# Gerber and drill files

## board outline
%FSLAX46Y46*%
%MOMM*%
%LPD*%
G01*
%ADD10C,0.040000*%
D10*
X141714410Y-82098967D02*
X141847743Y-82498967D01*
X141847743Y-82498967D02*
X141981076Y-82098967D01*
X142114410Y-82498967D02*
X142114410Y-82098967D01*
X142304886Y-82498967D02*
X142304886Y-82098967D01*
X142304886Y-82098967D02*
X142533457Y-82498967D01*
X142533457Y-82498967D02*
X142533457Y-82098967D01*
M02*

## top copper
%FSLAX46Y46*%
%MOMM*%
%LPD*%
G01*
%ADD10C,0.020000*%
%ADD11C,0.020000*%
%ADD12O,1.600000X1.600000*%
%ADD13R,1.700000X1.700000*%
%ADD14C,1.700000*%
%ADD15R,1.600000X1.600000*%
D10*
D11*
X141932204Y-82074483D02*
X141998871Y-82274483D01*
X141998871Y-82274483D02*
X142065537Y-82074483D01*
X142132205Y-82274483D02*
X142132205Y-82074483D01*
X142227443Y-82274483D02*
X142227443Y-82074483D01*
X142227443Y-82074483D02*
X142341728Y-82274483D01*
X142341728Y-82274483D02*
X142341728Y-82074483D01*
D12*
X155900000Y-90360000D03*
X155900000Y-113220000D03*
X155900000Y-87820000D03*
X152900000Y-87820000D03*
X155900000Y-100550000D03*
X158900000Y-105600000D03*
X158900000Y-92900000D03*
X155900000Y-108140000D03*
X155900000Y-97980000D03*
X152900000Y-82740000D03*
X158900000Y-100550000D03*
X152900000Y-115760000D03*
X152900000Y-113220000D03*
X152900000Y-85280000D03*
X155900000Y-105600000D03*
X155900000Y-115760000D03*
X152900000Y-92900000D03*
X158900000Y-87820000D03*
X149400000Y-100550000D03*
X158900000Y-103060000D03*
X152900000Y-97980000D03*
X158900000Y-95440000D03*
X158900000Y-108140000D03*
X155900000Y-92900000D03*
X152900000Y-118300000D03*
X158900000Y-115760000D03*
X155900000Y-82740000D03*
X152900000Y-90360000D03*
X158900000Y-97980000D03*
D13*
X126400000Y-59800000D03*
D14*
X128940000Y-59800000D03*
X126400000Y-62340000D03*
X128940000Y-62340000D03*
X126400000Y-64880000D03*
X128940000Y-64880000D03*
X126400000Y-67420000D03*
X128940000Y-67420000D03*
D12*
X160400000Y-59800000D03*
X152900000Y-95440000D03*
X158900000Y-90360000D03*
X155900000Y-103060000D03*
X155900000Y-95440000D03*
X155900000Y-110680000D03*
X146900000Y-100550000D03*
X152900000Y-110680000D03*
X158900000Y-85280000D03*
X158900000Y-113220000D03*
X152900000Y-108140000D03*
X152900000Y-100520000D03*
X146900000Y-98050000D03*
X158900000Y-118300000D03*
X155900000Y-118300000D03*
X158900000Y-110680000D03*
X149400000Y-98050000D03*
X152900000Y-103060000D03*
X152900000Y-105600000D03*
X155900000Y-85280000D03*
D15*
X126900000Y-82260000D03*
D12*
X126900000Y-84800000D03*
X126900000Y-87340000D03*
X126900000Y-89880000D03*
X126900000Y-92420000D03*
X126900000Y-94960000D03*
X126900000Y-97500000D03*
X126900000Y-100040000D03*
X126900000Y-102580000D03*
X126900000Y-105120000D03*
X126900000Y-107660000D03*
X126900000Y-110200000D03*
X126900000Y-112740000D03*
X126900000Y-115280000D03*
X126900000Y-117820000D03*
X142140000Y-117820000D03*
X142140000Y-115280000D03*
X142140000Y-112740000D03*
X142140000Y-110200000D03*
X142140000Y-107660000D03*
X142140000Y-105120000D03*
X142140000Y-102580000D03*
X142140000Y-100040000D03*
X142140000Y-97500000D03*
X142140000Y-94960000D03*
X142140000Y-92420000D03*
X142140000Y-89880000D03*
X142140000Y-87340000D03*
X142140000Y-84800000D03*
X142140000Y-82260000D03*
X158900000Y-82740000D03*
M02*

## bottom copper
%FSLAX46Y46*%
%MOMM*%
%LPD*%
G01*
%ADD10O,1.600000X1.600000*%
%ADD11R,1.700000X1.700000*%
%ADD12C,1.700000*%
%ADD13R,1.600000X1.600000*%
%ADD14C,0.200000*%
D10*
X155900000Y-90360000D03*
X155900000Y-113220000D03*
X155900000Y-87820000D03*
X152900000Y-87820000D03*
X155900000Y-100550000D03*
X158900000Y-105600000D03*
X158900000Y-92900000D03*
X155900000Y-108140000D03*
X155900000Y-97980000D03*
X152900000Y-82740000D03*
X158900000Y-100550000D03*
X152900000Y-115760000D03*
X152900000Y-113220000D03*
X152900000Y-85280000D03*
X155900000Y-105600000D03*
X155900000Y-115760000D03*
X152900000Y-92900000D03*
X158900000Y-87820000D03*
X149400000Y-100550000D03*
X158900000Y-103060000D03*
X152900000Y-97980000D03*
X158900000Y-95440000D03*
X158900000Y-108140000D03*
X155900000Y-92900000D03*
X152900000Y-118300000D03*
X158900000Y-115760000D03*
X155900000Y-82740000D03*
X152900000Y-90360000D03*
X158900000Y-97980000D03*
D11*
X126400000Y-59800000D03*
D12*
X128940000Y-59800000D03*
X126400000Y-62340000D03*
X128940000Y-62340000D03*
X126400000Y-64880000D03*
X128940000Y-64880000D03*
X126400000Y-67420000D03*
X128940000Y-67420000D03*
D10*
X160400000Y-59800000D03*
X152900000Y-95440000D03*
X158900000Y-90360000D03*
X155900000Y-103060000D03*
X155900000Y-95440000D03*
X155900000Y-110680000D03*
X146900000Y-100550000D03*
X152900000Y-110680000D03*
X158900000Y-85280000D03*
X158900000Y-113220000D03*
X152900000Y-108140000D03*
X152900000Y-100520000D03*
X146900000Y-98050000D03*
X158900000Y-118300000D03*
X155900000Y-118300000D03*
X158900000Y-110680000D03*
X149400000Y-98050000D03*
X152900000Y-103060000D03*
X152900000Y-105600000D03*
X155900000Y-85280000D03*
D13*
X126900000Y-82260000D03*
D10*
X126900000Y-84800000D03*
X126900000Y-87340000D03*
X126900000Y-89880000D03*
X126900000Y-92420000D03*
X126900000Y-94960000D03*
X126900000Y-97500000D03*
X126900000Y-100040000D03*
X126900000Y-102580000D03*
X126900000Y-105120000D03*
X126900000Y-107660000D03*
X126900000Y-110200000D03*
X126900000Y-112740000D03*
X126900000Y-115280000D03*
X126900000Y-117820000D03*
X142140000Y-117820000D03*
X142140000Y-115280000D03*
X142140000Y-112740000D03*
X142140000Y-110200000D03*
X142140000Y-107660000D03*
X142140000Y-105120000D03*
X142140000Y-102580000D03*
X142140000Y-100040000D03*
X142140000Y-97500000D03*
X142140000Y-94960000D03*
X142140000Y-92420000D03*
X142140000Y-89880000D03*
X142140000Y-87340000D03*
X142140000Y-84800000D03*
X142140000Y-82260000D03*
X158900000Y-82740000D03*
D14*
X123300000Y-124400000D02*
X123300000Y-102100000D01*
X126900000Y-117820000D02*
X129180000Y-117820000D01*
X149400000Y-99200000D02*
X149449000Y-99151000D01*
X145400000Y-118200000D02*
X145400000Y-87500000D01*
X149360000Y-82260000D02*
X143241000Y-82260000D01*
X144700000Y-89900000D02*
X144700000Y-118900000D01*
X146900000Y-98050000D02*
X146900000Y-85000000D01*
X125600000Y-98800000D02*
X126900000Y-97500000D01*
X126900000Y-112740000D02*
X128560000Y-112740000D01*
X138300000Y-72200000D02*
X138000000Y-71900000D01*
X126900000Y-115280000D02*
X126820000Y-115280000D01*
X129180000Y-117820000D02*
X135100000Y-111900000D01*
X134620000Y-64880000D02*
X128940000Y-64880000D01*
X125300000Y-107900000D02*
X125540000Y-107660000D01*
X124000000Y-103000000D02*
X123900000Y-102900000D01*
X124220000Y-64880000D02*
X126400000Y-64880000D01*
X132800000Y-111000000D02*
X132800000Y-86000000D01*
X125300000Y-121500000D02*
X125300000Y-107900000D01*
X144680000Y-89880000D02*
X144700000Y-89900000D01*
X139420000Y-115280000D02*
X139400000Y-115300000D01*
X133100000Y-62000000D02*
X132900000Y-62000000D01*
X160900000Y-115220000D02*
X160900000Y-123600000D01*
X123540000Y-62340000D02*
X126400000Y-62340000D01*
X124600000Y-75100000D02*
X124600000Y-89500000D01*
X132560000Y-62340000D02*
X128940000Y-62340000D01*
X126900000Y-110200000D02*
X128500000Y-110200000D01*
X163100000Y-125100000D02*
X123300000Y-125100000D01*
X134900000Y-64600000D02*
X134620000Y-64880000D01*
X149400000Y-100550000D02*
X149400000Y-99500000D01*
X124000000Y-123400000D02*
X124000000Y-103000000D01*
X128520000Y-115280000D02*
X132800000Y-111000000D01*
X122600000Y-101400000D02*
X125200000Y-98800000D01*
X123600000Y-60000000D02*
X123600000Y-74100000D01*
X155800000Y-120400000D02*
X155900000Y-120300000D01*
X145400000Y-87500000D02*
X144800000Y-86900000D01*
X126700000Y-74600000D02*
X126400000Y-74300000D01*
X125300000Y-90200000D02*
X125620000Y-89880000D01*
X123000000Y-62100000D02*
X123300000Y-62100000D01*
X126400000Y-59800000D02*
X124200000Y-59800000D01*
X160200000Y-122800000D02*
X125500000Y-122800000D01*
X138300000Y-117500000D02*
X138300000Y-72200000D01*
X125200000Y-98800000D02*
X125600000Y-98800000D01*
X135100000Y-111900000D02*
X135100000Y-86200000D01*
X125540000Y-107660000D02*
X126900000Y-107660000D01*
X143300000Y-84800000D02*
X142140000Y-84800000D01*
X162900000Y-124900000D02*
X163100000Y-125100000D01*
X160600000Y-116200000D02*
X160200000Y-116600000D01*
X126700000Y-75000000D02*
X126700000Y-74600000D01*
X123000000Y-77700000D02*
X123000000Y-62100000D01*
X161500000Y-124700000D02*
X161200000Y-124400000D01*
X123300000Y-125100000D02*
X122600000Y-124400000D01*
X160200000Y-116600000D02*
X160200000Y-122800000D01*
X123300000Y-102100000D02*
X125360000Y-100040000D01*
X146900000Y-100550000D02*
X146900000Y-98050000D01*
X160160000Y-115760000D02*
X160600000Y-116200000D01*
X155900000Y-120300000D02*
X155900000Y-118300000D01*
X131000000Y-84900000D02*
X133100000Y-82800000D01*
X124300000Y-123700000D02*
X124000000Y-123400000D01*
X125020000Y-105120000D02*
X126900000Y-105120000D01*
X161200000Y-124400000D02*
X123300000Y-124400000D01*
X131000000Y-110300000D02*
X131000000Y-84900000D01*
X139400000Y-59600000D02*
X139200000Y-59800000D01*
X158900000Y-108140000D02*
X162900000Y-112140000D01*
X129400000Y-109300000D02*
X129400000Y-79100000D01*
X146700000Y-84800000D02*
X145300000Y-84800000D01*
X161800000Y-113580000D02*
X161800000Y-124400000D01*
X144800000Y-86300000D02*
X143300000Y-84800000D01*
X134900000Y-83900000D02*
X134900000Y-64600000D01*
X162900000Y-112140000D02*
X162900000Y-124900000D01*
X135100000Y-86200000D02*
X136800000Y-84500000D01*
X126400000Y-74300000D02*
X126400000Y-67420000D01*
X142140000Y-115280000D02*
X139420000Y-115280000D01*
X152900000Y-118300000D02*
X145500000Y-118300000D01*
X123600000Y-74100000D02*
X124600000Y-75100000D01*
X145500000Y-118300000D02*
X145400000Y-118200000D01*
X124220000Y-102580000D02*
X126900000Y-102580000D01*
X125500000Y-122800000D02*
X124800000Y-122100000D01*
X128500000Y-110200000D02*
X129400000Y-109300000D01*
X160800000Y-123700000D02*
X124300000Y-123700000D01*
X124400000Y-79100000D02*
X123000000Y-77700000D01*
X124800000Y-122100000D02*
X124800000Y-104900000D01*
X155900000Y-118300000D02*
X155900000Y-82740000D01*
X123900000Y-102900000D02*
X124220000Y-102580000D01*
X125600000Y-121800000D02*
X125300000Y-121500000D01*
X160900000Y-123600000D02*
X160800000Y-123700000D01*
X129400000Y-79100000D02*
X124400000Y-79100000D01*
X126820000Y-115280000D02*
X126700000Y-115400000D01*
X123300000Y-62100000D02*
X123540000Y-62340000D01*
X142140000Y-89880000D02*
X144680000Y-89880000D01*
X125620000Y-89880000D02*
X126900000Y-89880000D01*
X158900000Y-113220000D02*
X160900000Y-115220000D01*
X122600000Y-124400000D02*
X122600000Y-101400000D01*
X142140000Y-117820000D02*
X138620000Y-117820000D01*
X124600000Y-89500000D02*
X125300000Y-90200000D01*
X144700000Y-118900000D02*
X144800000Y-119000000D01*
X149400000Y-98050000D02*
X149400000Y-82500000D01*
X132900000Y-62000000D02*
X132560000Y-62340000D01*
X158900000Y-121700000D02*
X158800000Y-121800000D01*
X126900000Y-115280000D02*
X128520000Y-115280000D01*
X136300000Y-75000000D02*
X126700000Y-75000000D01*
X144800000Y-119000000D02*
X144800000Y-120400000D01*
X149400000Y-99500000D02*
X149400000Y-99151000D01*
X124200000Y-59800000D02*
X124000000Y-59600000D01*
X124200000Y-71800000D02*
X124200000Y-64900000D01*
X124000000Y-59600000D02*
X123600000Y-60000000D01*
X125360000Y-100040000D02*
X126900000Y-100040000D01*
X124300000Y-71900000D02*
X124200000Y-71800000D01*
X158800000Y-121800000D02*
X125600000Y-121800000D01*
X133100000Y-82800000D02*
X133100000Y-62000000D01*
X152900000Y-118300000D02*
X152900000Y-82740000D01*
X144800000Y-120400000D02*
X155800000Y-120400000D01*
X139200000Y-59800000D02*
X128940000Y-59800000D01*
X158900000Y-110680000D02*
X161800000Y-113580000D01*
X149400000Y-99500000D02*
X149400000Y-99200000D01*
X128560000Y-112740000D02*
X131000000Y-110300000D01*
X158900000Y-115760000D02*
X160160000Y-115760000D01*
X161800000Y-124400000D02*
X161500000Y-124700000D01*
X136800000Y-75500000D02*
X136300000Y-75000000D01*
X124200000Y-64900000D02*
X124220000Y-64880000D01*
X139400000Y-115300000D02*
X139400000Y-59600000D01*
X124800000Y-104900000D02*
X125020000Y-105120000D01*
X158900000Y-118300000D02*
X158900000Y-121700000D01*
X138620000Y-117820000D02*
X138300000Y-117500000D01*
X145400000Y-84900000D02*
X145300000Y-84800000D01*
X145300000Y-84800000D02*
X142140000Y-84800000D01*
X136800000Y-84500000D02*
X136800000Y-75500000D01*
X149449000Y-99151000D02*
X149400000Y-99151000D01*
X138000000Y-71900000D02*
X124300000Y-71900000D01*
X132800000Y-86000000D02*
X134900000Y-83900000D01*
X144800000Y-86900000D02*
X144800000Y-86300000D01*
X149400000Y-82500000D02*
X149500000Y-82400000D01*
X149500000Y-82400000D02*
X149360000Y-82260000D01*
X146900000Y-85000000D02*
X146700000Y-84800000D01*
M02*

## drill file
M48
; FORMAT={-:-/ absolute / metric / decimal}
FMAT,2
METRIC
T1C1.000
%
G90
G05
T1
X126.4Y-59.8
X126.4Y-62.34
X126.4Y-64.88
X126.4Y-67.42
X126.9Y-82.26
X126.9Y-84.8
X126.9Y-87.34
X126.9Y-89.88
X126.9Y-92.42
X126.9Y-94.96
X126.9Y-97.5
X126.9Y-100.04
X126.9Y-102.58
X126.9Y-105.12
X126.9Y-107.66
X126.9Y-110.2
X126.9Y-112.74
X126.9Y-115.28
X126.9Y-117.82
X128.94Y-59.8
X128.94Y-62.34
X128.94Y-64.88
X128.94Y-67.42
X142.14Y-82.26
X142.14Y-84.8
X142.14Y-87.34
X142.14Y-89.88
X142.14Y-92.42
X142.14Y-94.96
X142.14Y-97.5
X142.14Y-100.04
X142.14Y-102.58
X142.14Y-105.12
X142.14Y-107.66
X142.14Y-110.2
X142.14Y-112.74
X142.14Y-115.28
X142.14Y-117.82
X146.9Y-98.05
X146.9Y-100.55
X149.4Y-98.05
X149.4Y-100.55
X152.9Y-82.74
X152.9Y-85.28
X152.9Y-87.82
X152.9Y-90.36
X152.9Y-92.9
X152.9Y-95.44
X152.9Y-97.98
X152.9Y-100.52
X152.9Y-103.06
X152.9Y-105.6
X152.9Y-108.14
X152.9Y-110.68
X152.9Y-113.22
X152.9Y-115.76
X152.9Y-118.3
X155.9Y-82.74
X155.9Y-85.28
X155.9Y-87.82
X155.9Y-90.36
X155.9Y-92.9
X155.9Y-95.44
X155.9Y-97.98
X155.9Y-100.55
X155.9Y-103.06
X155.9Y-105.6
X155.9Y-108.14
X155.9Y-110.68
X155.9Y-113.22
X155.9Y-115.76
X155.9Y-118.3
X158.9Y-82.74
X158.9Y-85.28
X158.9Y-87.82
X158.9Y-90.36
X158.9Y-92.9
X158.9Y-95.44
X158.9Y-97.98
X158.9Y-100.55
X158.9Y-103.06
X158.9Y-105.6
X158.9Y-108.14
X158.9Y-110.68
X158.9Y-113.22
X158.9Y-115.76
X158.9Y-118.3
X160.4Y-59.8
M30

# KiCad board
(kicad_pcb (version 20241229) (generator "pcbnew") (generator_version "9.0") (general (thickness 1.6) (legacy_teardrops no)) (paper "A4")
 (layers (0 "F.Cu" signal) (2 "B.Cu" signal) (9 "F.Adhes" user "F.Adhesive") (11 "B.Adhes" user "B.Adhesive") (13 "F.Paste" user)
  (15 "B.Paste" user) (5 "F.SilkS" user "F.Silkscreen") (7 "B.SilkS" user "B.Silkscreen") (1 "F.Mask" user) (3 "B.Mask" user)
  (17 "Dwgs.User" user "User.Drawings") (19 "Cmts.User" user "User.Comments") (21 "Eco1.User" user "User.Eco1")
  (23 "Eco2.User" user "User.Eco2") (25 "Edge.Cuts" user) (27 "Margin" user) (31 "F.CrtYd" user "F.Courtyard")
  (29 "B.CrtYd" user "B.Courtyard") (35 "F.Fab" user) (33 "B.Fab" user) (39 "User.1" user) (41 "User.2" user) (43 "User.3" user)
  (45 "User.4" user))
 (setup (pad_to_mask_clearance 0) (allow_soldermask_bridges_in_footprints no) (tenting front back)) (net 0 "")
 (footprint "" (layer "F.Cu") (at 155.9 90.36)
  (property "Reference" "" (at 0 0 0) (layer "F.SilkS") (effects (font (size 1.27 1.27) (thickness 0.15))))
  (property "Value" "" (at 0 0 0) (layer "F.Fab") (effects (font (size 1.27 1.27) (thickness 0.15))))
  (pad "27" thru_hole oval (at 0 0) (size 1.6 1.6) (drill 1) (layers "*.Cu" "*.Mask") (remove_unused_layers no)))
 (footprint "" (layer "F.Cu") (at 155.9 113.22)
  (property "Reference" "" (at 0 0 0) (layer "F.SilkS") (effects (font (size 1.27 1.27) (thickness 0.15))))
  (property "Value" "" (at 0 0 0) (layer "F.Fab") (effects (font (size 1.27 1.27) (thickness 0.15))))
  (pad "18" thru_hole oval (at 0 0) (size 1.6 1.6) (drill 1) (layers "*.Cu" "*.Mask") (remove_unused_layers no)))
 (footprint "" (layer "F.Cu") (at 155.9 87.82)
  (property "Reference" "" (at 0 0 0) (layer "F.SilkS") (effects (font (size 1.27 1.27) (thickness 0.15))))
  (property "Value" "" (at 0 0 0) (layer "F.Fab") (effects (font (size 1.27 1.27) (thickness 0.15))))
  (pad "28" thru_hole oval (at 0 0) (size 1.6 1.6) (drill 1) (layers "*.Cu" "*.Mask") (remove_unused_layers no)))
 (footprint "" (layer "F.Cu") (at 152.9 87.82)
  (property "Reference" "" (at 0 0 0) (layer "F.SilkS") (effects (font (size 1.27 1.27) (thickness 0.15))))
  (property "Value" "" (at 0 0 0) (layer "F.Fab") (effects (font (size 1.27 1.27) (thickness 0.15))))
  (pad "28" thru_hole oval (at 0 0) (size 1.6 1.6) (drill 1) (layers "*.Cu" "*.Mask") (remove_unused_layers no)))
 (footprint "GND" (layer "F.Cu") (at 155.9 100.55)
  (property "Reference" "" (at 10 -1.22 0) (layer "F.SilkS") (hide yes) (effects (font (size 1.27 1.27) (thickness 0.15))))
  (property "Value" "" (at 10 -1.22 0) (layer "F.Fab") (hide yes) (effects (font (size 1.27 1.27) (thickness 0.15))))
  (pad "23" thru_hole oval (at 0 0) (size 1.6 1.6) (drill 1) (layers "*.Cu" "*.Mask") (remove_unused_layers no)))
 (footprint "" (layer "F.Cu") (at 158.9 105.6)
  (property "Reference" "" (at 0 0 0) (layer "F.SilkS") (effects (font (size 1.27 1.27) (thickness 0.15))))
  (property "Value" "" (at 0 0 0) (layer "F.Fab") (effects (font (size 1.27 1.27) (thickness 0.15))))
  (pad "21" thru_hole oval (at 0 0) (size 1.6 1.6) (drill 1) (layers "*.Cu" "*.Mask") (remove_unused_layers no)))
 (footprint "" (layer "F.Cu") (at 158.9 92.9)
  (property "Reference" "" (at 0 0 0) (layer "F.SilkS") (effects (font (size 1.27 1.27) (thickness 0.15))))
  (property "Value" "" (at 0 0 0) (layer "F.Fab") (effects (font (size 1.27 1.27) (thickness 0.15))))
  (pad "26" thru_hole oval (at 0 0) (size 1.6 1.6) (drill 1) (layers "*.Cu" "*.Mask") (remove_unused_layers no)))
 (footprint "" (layer "F.Cu") (at 155.9 108.14)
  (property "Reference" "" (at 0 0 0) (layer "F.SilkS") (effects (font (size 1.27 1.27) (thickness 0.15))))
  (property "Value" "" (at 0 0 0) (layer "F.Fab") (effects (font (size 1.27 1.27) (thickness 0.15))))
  (pad "20" thru_hole oval (at 0 0) (size 1.6 1.6) (drill 1) (layers "*.Cu" "*.Mask") (remove_unused_layers no)))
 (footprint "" (layer "F.Cu") (at 155.9 97.98)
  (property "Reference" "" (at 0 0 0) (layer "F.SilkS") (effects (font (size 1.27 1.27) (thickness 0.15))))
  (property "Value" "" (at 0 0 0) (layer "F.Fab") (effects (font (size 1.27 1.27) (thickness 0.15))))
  (pad "24" thru_hole oval (at 0 0) (size 1.6 1.6) (drill 1) (layers "*.Cu" "*.Mask") (remove_unused_layers no)))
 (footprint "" (layer "F.Cu") (at 152.9 82.74)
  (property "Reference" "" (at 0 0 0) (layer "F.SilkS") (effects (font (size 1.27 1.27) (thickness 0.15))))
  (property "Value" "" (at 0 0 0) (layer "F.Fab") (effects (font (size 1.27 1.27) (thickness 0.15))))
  (pad "30" thru_hole oval (at 0 0) (size 1.6 1.6) (drill 1) (layers "*.Cu" "*.Mask") (remove_unused_layers no)))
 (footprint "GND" (layer "F.Cu") (at 158.9 100.55)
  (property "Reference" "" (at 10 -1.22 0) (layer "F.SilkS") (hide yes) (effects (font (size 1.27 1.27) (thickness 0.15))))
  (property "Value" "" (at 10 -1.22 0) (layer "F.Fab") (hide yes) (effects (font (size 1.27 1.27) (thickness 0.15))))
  (pad "23" thru_hole oval (at 0 0) (size 1.6 1.6) (drill 1) (layers "*.Cu" "*.Mask") (remove_unused_layers no)))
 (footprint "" (layer "F.Cu") (at 152.9 115.76)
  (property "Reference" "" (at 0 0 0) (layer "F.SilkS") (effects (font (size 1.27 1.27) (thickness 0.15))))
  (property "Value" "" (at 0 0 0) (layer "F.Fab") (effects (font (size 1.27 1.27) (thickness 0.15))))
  (pad "17" thru_hole oval (at 0 0) (size 1.6 1.6) (drill 1) (layers "*.Cu" "*.Mask") (remove_unused_layers no)))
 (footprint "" (layer "F.Cu") (at 152.9 113.22)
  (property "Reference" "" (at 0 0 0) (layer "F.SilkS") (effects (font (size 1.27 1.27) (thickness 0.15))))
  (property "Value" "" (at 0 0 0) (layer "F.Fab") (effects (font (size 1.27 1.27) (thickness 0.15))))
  (pad "18" thru_hole oval (at 0 0) (size 1.6 1.6) (drill 1) (layers "*.Cu" "*.Mask") (remove_unused_layers no)))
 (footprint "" (layer "F.Cu") (at 152.9 85.28)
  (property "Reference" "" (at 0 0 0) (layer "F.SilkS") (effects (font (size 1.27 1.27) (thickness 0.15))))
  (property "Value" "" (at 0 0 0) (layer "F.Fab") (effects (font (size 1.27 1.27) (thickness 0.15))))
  (pad "29" thru_hole oval (at 0 0) (size 1.6 1.6) (drill 1) (layers "*.Cu" "*.Mask") (remove_unused_layers no)))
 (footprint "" (layer "F.Cu") (at 155.9 105.6)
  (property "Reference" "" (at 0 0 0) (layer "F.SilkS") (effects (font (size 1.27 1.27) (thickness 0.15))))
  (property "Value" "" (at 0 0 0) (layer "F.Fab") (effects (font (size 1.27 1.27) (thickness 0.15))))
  (pad "21" thru_hole oval (at 0 0) (size 1.6 1.6) (drill 1) (layers "*.Cu" "*.Mask") (remove_unused_layers no)))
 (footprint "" (layer "F.Cu") (at 155.9 115.76)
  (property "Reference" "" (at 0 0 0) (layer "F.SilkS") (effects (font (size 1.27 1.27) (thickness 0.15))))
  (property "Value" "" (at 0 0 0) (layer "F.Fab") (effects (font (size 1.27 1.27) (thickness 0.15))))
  (pad "17" thru_hole oval (at 0 0) (size 1.6 1.6) (drill 1) (layers "*.Cu" "*.Mask") (remove_unused_layers no)))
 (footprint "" (layer "F.Cu") (at 152.9 92.9)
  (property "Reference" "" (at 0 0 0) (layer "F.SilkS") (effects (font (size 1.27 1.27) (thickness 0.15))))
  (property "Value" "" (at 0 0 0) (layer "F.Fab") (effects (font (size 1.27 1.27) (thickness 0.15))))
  (pad "26" thru_hole oval (at 0 0) (size 1.6 1.6) (drill 1) (layers "*.Cu" "*.Mask") (remove_unused_layers no)))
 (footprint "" (layer "F.Cu") (at 158.9 87.82)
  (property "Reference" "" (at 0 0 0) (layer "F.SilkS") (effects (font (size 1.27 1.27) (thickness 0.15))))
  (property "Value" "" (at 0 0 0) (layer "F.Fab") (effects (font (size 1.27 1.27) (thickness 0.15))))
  (pad "28" thru_hole oval (at 0 0) (size 1.6 1.6) (drill 1) (layers "*.Cu" "*.Mask") (remove_unused_layers no)))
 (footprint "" (layer "F.Cu") (at 149.4 100.55)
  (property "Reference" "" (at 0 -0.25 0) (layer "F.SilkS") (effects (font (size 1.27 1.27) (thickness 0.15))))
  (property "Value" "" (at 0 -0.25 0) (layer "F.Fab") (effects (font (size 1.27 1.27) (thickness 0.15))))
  (pad "30" thru_hole oval (at 0 0) (size 1.6 1.6) (drill 1) (layers "*.Cu" "*.Mask") (remove_unused_layers no)))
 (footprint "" (layer "F.Cu") (at 158.9 103.06)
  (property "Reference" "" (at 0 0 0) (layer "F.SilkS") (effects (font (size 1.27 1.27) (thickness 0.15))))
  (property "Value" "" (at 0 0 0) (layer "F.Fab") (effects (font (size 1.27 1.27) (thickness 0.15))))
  (pad "22" thru_hole oval (at 0 0) (size 1.6 1.6) (drill 1) (layers "*.Cu" "*.Mask") (remove_unused_layers no)))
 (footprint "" (layer "F.Cu") (at 152.9 97.98)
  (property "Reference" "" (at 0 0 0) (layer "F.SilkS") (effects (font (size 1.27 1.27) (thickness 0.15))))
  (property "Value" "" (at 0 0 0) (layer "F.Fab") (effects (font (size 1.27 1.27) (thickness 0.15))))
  (pad "24" thru_hole oval (at 0 0) (size 1.6 1.6) (drill 1) (layers "*.Cu" "*.Mask") (remove_unused_layers no)))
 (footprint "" (layer "F.Cu") (at 158.9 95.44)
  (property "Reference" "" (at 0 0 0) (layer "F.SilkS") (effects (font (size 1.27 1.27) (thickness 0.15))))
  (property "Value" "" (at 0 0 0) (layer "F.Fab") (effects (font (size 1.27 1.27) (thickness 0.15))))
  (pad "25" thru_hole oval (at 0 0) (size 1.6 1.6) (drill 1) (layers "*.Cu" "*.Mask") (remove_unused_layers no)))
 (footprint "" (layer "F.Cu") (at 158.9 108.14)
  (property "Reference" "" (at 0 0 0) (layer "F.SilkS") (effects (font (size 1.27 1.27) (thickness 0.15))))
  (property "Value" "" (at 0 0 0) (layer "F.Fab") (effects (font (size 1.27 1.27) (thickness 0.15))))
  (pad "20" thru_hole oval (at 0 0) (size 1.6 1.6) (drill 1) (layers "*.Cu" "*.Mask") (remove_unused_layers no)))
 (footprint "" (layer "F.Cu") (at 155.9 92.9)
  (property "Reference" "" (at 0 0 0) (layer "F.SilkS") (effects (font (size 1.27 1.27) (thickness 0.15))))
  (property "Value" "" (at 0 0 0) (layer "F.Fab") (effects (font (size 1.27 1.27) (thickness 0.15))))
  (pad "26" thru_hole oval (at 0 0) (size 1.6 1.6) (drill 1) (layers "*.Cu" "*.Mask") (remove_unused_layers no)))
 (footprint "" (layer "F.Cu") (at 152.9 118.3)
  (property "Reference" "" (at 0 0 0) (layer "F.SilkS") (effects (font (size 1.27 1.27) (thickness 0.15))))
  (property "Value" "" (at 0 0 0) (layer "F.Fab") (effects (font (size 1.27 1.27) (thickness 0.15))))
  (pad "16" thru_hole oval (at 0 0) (size 1.6 1.6) (drill 1) (layers "*.Cu" "*.Mask") (remove_unused_layers no)))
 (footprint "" (layer "F.Cu") (at 158.9 115.76)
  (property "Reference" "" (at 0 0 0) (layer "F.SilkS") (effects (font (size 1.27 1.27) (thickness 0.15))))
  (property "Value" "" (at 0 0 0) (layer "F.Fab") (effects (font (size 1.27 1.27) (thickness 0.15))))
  (pad "17" thru_hole oval (at 0 0) (size 1.6 1.6) (drill 1) (layers "*.Cu" "*.Mask") (remove_unused_layers no)))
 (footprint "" (layer "F.Cu") (at 155.9 82.74)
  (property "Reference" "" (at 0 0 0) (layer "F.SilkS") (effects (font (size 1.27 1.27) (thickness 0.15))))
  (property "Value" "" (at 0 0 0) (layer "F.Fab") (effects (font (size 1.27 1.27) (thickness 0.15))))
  (pad "30" thru_hole oval (at 0 0) (size 1.6 1.6) (drill 1) (layers "*.Cu" "*.Mask") (remove_unused_layers no)))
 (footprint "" (layer "F.Cu") (at 152.9 90.36)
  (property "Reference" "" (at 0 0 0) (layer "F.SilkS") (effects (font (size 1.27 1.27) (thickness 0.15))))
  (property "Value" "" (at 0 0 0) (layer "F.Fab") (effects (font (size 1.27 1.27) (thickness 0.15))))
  (pad "27" thru_hole oval (at 0 0) (size 1.6 1.6) (drill 1) (layers "*.Cu" "*.Mask") (remove_unused_layers no)))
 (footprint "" (layer "F.Cu") (at 158.9 97.98)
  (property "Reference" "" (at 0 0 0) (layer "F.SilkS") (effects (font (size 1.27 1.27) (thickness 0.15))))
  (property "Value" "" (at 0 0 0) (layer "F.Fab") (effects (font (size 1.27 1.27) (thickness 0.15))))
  (pad "24" thru_hole oval (at 0 0) (size 1.6 1.6) (drill 1) (layers "*.Cu" "*.Mask") (remove_unused_layers no)))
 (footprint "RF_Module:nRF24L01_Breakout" (layer "F.Cu") (at 126.4 59.8)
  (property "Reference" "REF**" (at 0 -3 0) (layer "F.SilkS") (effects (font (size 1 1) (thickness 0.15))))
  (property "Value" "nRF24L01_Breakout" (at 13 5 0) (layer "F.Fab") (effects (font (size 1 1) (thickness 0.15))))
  (pad "1" thru_hole rect (at 0 0) (size 1.7 1.7) (drill 1) (layers "*.Cu" "*.Mask") (remove_unused_layers no))
  (pad "2" thru_hole circle (at 2.54 0) (size 1.7 1.7) (drill 1) (layers "*.Cu" "*.Mask") (remove_unused_layers no))
  (pad "3" thru_hole circle (at 0 2.54) (size 1.7 1.7) (drill 1) (layers "*.Cu" "*.Mask") (remove_unused_layers no))
  (pad "4" thru_hole circle (at 2.54 2.54) (size 1.7 1.7) (drill 1) (layers "*.Cu" "*.Mask") (remove_unused_layers no))
  (pad "5" thru_hole circle (at 0 5.08) (size 1.7 1.7) (drill 1) (layers "*.Cu" "*.Mask") (remove_unused_layers no))
  (pad "6" thru_hole circle (at 2.54 5.08) (size 1.7 1.7) (drill 1) (layers "*.Cu" "*.Mask") (remove_unused_layers no))
  (pad "7" thru_hole circle (at 0 7.62) (size 1.7 1.7) (drill 1) (layers "*.Cu" "*.Mask") (remove_unused_layers no))
  (pad "8" thru_hole circle (at 2.54 7.62) (size 1.7 1.7) (drill 1) (layers "*.Cu" "*.Mask") (remove_unused_layers no)))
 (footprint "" (layer "F.Cu") (at 160.4 59.8)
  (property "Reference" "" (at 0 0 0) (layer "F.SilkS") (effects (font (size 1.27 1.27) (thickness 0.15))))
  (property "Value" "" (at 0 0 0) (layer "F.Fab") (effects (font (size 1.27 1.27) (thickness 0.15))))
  (pad "30" thru_hole oval (at 0 0) (size 1.6 1.6) (drill 1) (layers "*.Cu" "*.Mask") (remove_unused_layers no)))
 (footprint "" (layer "F.Cu") (at 152.9 95.44)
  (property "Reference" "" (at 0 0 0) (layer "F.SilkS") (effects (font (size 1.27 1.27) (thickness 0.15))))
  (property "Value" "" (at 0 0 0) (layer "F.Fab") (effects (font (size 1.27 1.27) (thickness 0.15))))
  (pad "25" thru_hole oval (at 0 0) (size 1.6 1.6) (drill 1) (layers "*.Cu" "*.Mask") (remove_unused_layers no)))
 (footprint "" (layer "F.Cu") (at 158.9 90.36)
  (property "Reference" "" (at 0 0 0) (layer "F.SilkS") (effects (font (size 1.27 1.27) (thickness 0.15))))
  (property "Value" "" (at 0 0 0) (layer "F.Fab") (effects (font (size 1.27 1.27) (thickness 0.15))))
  (pad "27" thru_hole oval (at 0 0) (size 1.6 1.6) (drill 1) (layers "*.Cu" "*.Mask") (remove_unused_layers no)))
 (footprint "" (layer "F.Cu") (at 155.9 103.06)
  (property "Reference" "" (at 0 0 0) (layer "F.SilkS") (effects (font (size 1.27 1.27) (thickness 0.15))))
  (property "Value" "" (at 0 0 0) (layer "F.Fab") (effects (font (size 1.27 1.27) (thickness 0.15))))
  (pad "22" thru_hole oval (at 0 0) (size 1.6 1.6) (drill 1) (layers "*.Cu" "*.Mask") (remove_unused_layers no)))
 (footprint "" (layer "F.Cu") (at 155.9 95.44)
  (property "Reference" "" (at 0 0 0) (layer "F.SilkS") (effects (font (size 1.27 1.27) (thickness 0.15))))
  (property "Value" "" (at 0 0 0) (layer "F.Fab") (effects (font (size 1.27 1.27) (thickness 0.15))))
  (pad "25" thru_hole oval (at 0 0) (size 1.6 1.6) (drill 1) (layers "*.Cu" "*.Mask") (remove_unused_layers no)))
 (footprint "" (layer "F.Cu") (at 155.9 110.68)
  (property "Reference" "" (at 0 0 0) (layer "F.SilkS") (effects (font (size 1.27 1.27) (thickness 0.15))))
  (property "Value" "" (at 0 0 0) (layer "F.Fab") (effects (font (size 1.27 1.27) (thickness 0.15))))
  (pad "19" thru_hole oval (at 0 0) (size 1.6 1.6) (drill 1) (layers "*.Cu" "*.Mask") (remove_unused_layers no)))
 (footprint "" (layer "F.Cu") (at 146.9 100.55)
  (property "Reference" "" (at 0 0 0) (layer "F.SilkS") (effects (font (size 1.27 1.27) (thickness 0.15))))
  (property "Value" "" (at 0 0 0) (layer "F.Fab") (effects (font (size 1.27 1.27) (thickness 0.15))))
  (pad "30" thru_hole oval (at 0 0) (size 1.6 1.6) (drill 1) (layers "*.Cu" "*.Mask") (remove_unused_layers no)))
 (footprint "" (layer "F.Cu") (at 152.9 110.68)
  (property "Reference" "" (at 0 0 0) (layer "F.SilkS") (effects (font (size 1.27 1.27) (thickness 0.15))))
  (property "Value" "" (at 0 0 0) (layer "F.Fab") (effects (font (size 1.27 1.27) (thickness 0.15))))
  (pad "19" thru_hole oval (at 0 0) (size 1.6 1.6) (drill 1) (layers "*.Cu" "*.Mask") (remove_unused_layers no)))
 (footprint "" (layer "F.Cu") (at 158.9 85.28)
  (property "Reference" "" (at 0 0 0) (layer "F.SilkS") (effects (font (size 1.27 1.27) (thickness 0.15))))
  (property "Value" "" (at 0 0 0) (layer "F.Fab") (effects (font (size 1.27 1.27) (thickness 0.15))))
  (pad "29" thru_hole oval (at 0 0) (size 1.6 1.6) (drill 1) (layers "*.Cu" "*.Mask") (remove_unused_layers no)))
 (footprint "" (layer "F.Cu") (at 158.9 113.22)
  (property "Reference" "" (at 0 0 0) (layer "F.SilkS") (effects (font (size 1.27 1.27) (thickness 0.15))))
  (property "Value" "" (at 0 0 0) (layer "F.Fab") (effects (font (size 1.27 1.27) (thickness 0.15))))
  (pad "18" thru_hole oval (at 0 0) (size 1.6 1.6) (drill 1) (layers "*.Cu" "*.Mask") (remove_unused_layers no)))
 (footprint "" (layer "F.Cu") (at 152.9 108.14)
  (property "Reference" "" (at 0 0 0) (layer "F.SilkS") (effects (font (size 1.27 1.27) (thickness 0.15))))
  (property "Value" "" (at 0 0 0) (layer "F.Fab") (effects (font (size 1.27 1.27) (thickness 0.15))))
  (pad "20" thru_hole oval (at 0 0) (size 1.6 1.6) (drill 1) (layers "*.Cu" "*.Mask") (remove_unused_layers no)))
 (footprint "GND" (layer "F.Cu") (at 152.9 100.52)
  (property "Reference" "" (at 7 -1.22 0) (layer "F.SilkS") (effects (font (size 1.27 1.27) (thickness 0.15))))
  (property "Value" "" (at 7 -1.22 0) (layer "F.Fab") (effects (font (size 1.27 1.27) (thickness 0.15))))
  (pad "23" thru_hole oval (at 0 0) (size 1.6 1.6) (drill 1) (layers "*.Cu" "*.Mask") (remove_unused_layers no)))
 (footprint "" (layer "F.Cu") (at 146.9 98.05)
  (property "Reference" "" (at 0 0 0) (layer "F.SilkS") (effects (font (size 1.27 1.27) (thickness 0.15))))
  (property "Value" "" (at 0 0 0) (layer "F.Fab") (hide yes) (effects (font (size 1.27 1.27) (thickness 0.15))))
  (pad "30" thru_hole oval (at 0 0) (size 1.6 1.6) (drill 1) (layers "*.Cu" "*.Mask") (remove_unused_layers no)))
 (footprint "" (layer "F.Cu") (at 158.9 118.3)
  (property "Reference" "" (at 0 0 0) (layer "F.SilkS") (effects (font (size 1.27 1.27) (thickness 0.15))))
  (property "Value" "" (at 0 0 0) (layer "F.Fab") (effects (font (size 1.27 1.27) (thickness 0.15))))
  (pad "16" thru_hole oval (at 0 0) (size 1.6 1.6) (drill 1) (layers "*.Cu" "*.Mask") (remove_unused_layers no)))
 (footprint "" (layer "F.Cu") (at 155.9 118.3)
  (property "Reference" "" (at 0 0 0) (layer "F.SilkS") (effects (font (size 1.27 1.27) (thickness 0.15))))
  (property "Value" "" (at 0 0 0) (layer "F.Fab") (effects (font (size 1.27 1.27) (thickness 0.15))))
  (pad "16" thru_hole oval (at 0 0) (size 1.6 1.6) (drill 1) (layers "*.Cu" "*.Mask") (remove_unused_layers no)))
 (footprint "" (layer "F.Cu") (at 158.9 110.68)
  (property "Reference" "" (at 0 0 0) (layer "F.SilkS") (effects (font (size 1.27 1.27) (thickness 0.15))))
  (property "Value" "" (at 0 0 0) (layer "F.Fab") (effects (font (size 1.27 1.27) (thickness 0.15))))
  (pad "19" thru_hole oval (at 0 0) (size 1.6 1.6) (drill 1) (layers "*.Cu" "*.Mask") (remove_unused_layers no)))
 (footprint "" (layer "F.Cu") (at 149.4 98.05)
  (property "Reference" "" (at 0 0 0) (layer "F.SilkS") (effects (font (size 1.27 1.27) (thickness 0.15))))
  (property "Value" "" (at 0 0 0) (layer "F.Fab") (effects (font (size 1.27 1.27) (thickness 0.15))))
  (pad "30" thru_hole oval (at 0 0) (size 1.6 1.6) (drill 1) (layers "*.Cu" "*.Mask") (remove_unused_layers no)))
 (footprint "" (layer "F.Cu") (at 152.9 103.06)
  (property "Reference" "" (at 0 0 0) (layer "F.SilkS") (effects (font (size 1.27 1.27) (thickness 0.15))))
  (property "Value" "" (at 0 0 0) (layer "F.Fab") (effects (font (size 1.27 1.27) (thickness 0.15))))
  (pad "22" thru_hole oval (at 0 0) (size 1.6 1.6) (drill 1) (layers "*.Cu" "*.Mask") (remove_unused_layers no)))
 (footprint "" (layer "F.Cu") (at 152.9 105.6)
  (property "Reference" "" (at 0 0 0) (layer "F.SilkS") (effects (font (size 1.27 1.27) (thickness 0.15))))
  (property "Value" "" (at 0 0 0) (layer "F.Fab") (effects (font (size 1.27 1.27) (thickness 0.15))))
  (pad "21" thru_hole oval (at 0 0) (size 1.6 1.6) (drill 1) (layers "*.Cu" "*.Mask") (remove_unused_layers no)))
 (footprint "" (layer "F.Cu") (at 155.9 85.28)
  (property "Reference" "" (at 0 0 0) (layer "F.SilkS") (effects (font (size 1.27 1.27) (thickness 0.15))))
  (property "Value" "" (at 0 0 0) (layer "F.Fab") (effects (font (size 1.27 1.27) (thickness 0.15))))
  (pad "29" thru_hole oval (at 0 0) (size 1.6 1.6) (drill 1) (layers "*.Cu" "*.Mask") (remove_unused_layers no)))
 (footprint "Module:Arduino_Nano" (layer "F.Cu") (at 126.9 82.26)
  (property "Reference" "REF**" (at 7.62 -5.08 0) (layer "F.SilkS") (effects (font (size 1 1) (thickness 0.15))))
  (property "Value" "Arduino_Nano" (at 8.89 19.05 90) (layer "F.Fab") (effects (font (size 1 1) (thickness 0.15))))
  (pad "1" thru_hole rect (at 0 0) (size 1.6 1.6) (drill 1) (layers "*.Cu" "*.Mask") (remove_unused_layers no))
  (pad "2" thru_hole oval (at 0 2.54) (size 1.6 1.6) (drill 1) (layers "*.Cu" "*.Mask") (remove_unused_layers no))
  (pad "3" thru_hole oval (at 0 5.08) (size 1.6 1.6) (drill 1) (layers "*.Cu" "*.Mask") (remove_unused_layers no))
  (pad "4" thru_hole oval (at 0 7.62) (size 1.6 1.6) (drill 1) (layers "*.Cu" "*.Mask") (remove_unused_layers no))
  (pad "5" thru_hole oval (at 0 10.16) (size 1.6 1.6) (drill 1) (layers "*.Cu" "*.Mask") (remove_unused_layers no))
  (pad "6" thru_hole oval (at 0 12.7) (size 1.6 1.6) (drill 1) (layers "*.Cu" "*.Mask") (remove_unused_layers no))
  (pad "7" thru_hole oval (at 0 15.24) (size 1.6 1.6) (drill 1) (layers "*.Cu" "*.Mask") (remove_unused_layers no))
  (pad "8" thru_hole oval (at 0 17.78) (size 1.6 1.6) (drill 1) (layers "*.Cu" "*.Mask") (remove_unused_layers no))
  (pad "9" thru_hole oval (at 0 20.32) (size 1.6 1.6) (drill 1) (layers "*.Cu" "*.Mask") (remove_unused_layers no))
  (pad "10" thru_hole oval (at 0 22.86) (size 1.6 1.6) (drill 1) (layers "*.Cu" "*.Mask") (remove_unused_layers no))
  (pad "11" thru_hole oval (at 0 25.4) (size 1.6 1.6) (drill 1) (layers "*.Cu" "*.Mask") (remove_unused_layers no))
  (pad "12" thru_hole oval (at 0 27.94) (size 1.6 1.6) (drill 1) (layers "*.Cu" "*.Mask") (remove_unused_layers no))
  (pad "13" thru_hole oval (at 0 30.48) (size 1.6 1.6) (drill 1) (layers "*.Cu" "*.Mask") (remove_unused_layers no))
  (pad "14" thru_hole oval (at 0 33.02) (size 1.6 1.6) (drill 1) (layers "*.Cu" "*.Mask") (remove_unused_layers no))
  (pad "15" thru_hole oval (at 0 35.56) (size 1.6 1.6) (drill 1) (layers "*.Cu" "*.Mask") (remove_unused_layers no))
  (pad "16" thru_hole oval (at 15.24 35.56) (size 1.6 1.6) (drill 1) (layers "*.Cu" "*.Mask") (remove_unused_layers no))
  (pad "17" thru_hole oval (at 15.24 33.02) (size 1.6 1.6) (drill 1) (layers "*.Cu" "*.Mask") (remove_unused_layers no))
  (pad "18" thru_hole oval (at 15.24 30.48) (size 1.6 1.6) (drill 1) (layers "*.Cu" "*.Mask") (remove_unused_layers no))
  (pad "19" thru_hole oval (at 15.24 27.94) (size 1.6 1.6) (drill 1) (layers "*.Cu" "*.Mask") (remove_unused_layers no))
  (pad "20" thru_hole oval (at 15.24 25.4) (size 1.6 1.6) (drill 1) (layers "*.Cu" "*.Mask") (remove_unused_layers no))
  (pad "21" thru_hole oval (at 15.24 22.86) (size 1.6 1.6) (drill 1) (layers "*.Cu" "*.Mask") (remove_unused_layers no))
  (pad "22" thru_hole oval (at 15.24 20.32) (size 1.6 1.6) (drill 1) (layers "*.Cu" "*.Mask") (remove_unused_layers no))
  (pad "23" thru_hole oval (at 15.24 17.78) (size 1.6 1.6) (drill 1) (layers "*.Cu" "*.Mask") (remove_unused_layers no))
  (pad "24" thru_hole oval (at 15.24 15.24) (size 1.6 1.6) (drill 1) (layers "*.Cu" "*.Mask") (remove_unused_layers no))
  (pad "25" thru_hole oval (at 15.24 12.7) (size 1.6 1.6) (drill 1) (layers "*.Cu" "*.Mask") (remove_unused_layers no))
  (pad "26" thru_hole oval (at 15.24 10.16) (size 1.6 1.6) (drill 1) (layers "*.Cu" "*.Mask") (remove_unused_layers no))
  (pad "27" thru_hole oval (at 15.24 7.62) (size 1.6 1.6) (drill 1) (layers "*.Cu" "*.Mask") (remove_unused_layers no))
  (pad "28" thru_hole oval (at 15.24 5.08) (size 1.6 1.6) (drill 1) (layers "*.Cu" "*.Mask") (remove_unused_layers no))
  (pad "29" thru_hole oval (at 15.24 2.54) (size 1.6 1.6) (drill 1) (layers "*.Cu" "*.Mask") (remove_unused_layers no))
  (pad "30" thru_hole oval (at 15.24 0) (size 1.6 1.6) (drill 1) (layers "*.Cu" "*.Mask") (remove_unused_layers no)))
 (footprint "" (layer "F.Cu") (at 158.9 82.74)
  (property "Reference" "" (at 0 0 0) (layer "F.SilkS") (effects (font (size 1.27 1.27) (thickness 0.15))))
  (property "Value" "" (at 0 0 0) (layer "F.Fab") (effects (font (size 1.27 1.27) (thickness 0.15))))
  (pad "30" thru_hole oval (at 0 0) (size 1.6 1.6) (drill 1) (layers "*.Cu" "*.Mask") (remove_unused_layers no)))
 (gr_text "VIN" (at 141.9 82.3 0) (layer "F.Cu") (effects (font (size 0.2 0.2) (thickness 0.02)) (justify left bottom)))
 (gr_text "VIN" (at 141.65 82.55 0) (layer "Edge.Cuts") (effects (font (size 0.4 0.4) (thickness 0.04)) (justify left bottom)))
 (segment (start 123.3 124.4) (end 123.3 102.1) (width 0.2) (layer "B.Cu") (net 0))
 (segment (start 126.9 117.82) (end 129.18 117.82) (width 0.2) (layer "B.Cu") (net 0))
 (segment (start 149.4 99.2) (end 149.449 99.151) (width 0.2) (layer "B.Cu") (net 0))
 (segment (start 145.4 118.2) (end 145.4 87.5) (width 0.2) (layer "B.Cu") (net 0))
 (segment (start 149.36 82.26) (end 143.241 82.26) (width 0.2) (layer "B.Cu") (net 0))
 (segment (start 144.7 89.9) (end 144.7 118.9) (width 0.2) (layer "B.Cu") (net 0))
 (segment (start 146.9 98.05) (end 146.9 85) (width 0.2) (layer "B.Cu") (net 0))
 (segment (start 125.6 98.8) (end 126.9 97.5) (width 0.2) (layer "B.Cu") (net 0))
 (segment (start 126.9 112.74) (end 128.56 112.74) (width 0.2) (layer "B.Cu") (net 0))
 (segment (start 138.3 72.2) (end 138 71.9) (width 0.2) (layer "B.Cu") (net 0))
 (segment (start 126.9 115.28) (end 126.82 115.28) (width 0.2) (layer "B.Cu") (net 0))
 (segment (start 129.18 117.82) (end 135.1 111.9) (width 0.2) (layer "B.Cu") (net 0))
 (segment (start 134.62 64.88) (end 128.94 64.88) (width 0.2) (layer "B.Cu") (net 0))
 (segment (start 125.3 107.9) (end 125.54 107.66) (width 0.2) (layer "B.Cu") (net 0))
 (segment (start 124 103) (end 123.9 102.9) (width 0.2) (layer "B.Cu") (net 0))
 (segment (start 124.22 64.88) (end 126.4 64.88) (width 0.2) (layer "B.Cu") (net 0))
 (segment (start 132.8 111) (end 132.8 86) (width 0.2) (layer "B.Cu") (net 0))
 (segment (start 125.3 121.5) (end 125.3 107.9) (width 0.2) (layer "B.Cu") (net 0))
 (segment (start 144.68 89.88) (end 144.7 89.9) (width 0.2) (layer "B.Cu") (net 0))
 (segment (start 139.42 115.28) (end 139.4 115.3) (width 0.2) (layer "B.Cu") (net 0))
 (segment (start 133.1 62) (end 132.9 62) (width 0.2) (layer "B.Cu") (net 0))
 (segment (start 160.9 115.22) (end 160.9 123.6) (width 0.2) (layer "B.Cu") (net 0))
 (segment (start 123.54 62.34) (end 126.4 62.34) (width 0.2) (layer "B.Cu") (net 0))
 (segment (start 124.6 75.1) (end 124.6 89.5) (width 0.2) (layer "B.Cu") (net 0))
 (segment (start 132.56 62.34) (end 128.94 62.34) (width 0.2) (layer "B.Cu") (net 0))
 (segment (start 126.9 110.2) (end 128.5 110.2) (width 0.2) (layer "B.Cu") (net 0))
 (segment (start 163.1 125.1) (end 123.3 125.1) (width 0.2) (layer "B.Cu") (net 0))
 (segment (start 134.9 64.6) (end 134.62 64.88) (width 0.2) (layer "B.Cu") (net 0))
 (segment (start 149.4 100.55) (end 149.4 99.5) (width 0.2) (layer "B.Cu") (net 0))
 (segment (start 124 123.4) (end 124 103) (width 0.2) (layer "B.Cu") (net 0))
 (segment (start 128.52 115.28) (end 132.8 111) (width 0.2) (layer "B.Cu") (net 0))
 (segment (start 122.6 101.4) (end 125.2 98.8) (width 0.2) (layer "B.Cu") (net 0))
 (segment (start 123.6 60) (end 123.6 74.1) (width 0.2) (layer "B.Cu") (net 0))
 (segment (start 155.8 120.4) (end 155.9 120.3) (width 0.2) (layer "B.Cu") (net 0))
 (segment (start 145.4 87.5) (end 144.8 86.9) (width 0.2) (layer "B.Cu") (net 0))
 (segment (start 126.7 74.6) (end 126.4 74.3) (width 0.2) (layer "B.Cu") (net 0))
 (segment (start 125.3 90.2) (end 125.62 89.88) (width 0.2) (layer "B.Cu") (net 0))
 (segment (start 123 62.1) (end 123.3 62.1) (width 0.2) (layer "B.Cu") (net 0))
 (segment (start 126.4 59.8) (end 124.2 59.8) (width 0.2) (layer "B.Cu") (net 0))
 (segment (start 160.2 122.8) (end 125.5 122.8) (width 0.2) (layer "B.Cu") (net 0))
 (segment (start 138.3 117.5) (end 138.3 72.2) (width 0.2) (layer "B.Cu") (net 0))
 (segment (start 125.2 98.8) (end 125.6 98.8) (width 0.2) (layer "B.Cu") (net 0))
 (segment (start 135.1 111.9) (end 135.1 86.2) (width 0.2) (layer "B.Cu") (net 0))
 (segment (start 125.54 107.66) (end 126.9 107.66) (width 0.2) (layer "B.Cu") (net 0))
 (segment (start 143.3 84.8) (end 142.14 84.8) (width 0.2) (layer "B.Cu") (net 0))
 (segment (start 162.9 124.9) (end 163.1 125.1) (width 0.2) (layer "B.Cu") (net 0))
 (segment (start 160.6 116.2) (end 160.2 116.6) (width 0.2) (layer "B.Cu") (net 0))
 (segment (start 126.7 75) (end 126.7 74.6) (width 0.2) (layer "B.Cu") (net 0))
 (segment (start 123 77.7) (end 123 62.1) (width 0.2) (layer "B.Cu") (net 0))
 (segment (start 161.5 124.7) (end 161.2 124.4) (width 0.2) (layer "B.Cu") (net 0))
 (segment (start 123.3 125.1) (end 122.6 124.4) (width 0.2) (layer "B.Cu") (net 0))
 (segment (start 160.2 116.6) (end 160.2 122.8) (width 0.2) (layer "B.Cu") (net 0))
 (segment (start 123.3 102.1) (end 125.36 100.04) (width 0.2) (layer "B.Cu") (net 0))
 (segment (start 146.9 100.55) (end 146.9 98.05) (width 0.2) (layer "B.Cu") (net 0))
 (segment (start 160.16 115.76) (end 160.6 116.2) (width 0.2) (layer "B.Cu") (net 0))
 (segment (start 155.9 120.3) (end 155.9 118.3) (width 0.2) (layer "B.Cu") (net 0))
 (segment (start 131 84.9) (end 133.1 82.8) (width 0.2) (layer "B.Cu") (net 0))
 (segment (start 124.3 123.7) (end 124 123.4) (width 0.2) (layer "B.Cu") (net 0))
 (segment (start 125.02 105.12) (end 126.9 105.12) (width 0.2) (layer "B.Cu") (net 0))
 (segment (start 161.2 124.4) (end 123.3 124.4) (width 0.2) (layer "B.Cu") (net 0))
 (segment (start 131 110.3) (end 131 84.9) (width 0.2) (layer "B.Cu") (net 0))
 (segment (start 139.4 59.6) (end 139.2 59.8) (width 0.2) (layer "B.Cu") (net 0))
 (segment (start 158.9 108.14) (end 162.9 112.14) (width 0.2) (layer "B.Cu") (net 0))
 (segment (start 129.4 109.3) (end 129.4 79.1) (width 0.2) (layer "B.Cu") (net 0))
 (segment (start 146.7 84.8) (end 145.3 84.8) (width 0.2) (layer "B.Cu") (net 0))
 (segment (start 161.8 113.58) (end 161.8 124.4) (width 0.2) (layer "B.Cu") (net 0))
 (segment (start 144.8 86.3) (end 143.3 84.8) (width 0.2) (layer "B.Cu") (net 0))
 (segment (start 134.9 83.9) (end 134.9 64.6) (width 0.2) (layer "B.Cu") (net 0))
 (segment (start 162.9 112.14) (end 162.9 124.9) (width 0.2) (layer "B.Cu") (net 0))
 (segment (start 135.1 86.2) (end 136.8 84.5) (width 0.2) (layer "B.Cu") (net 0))
 (segment (start 126.4 74.3) (end 126.4 67.42) (width 0.2) (layer "B.Cu") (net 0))
 (segment (start 142.14 115.28) (end 139.42 115.28) (width 0.2) (layer "B.Cu") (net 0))
 (segment (start 152.9 118.3) (end 145.5 118.3) (width 0.2) (layer "B.Cu") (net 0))
 (segment (start 123.6 74.1) (end 124.6 75.1) (width 0.2) (layer "B.Cu") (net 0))
 (segment (start 145.5 118.3) (end 145.4 118.2) (width 0.2) (layer "B.Cu") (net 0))
 (segment (start 124.22 102.58) (end 126.9 102.58) (width 0.2) (layer "B.Cu") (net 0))
 (segment (start 125.5 122.8) (end 124.8 122.1) (width 0.2) (layer "B.Cu") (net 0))
 (segment (start 128.5 110.2) (end 129.4 109.3) (width 0.2) (layer "B.Cu") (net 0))
 (segment (start 160.8 123.7) (end 124.3 123.7) (width 0.2) (layer "B.Cu") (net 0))
 (segment (start 124.4 79.1) (end 123 77.7) (width 0.2) (layer "B.Cu") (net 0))
 (segment (start 124.8 122.1) (end 124.8 104.9) (width 0.2) (layer "B.Cu") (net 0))
 (segment (start 155.9 118.3) (end 155.9 82.74) (width 0.2) (layer "B.Cu") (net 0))
 (segment (start 123.9 102.9) (end 124.22 102.58) (width 0.2) (layer "B.Cu") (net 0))
 (segment (start 125.6 121.8) (end 125.3 121.5) (width 0.2) (layer "B.Cu") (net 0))
 (segment (start 160.9 123.6) (end 160.8 123.7) (width 0.2) (layer "B.Cu") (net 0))
 (segment (start 129.4 79.1) (end 124.4 79.1) (width 0.2) (layer "B.Cu") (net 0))
 (segment (start 126.82 115.28) (end 126.7 115.4) (width 0.2) (layer "B.Cu") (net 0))
 (segment (start 123.3 62.1) (end 123.54 62.34) (width 0.2) (layer "B.Cu") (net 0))
 (segment (start 142.14 89.88) (end 144.68 89.88) (width 0.2) (layer "B.Cu") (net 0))
 (segment (start 125.62 89.88) (end 126.9 89.88) (width 0.2) (layer "B.Cu") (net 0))
 (segment (start 158.9 113.22) (end 160.9 115.22) (width 0.2) (layer "B.Cu") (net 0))
 (segment (start 122.6 124.4) (end 122.6 101.4) (width 0.2) (layer "B.Cu") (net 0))
 (segment (start 142.14 117.82) (end 138.62 117.82) (width 0.2) (layer "B.Cu") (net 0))
 (segment (start 124.6 89.5) (end 125.3 90.2) (width 0.2) (layer "B.Cu") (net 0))
 (segment (start 144.7 118.9) (end 144.8 119) (width 0.2) (layer "B.Cu") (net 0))
 (segment (start 149.4 98.05) (end 149.4 82.5) (width 0.2) (layer "B.Cu") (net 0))
 (segment (start 132.9 62) (end 132.56 62.34) (width 0.2) (layer "B.Cu") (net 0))
 (segment (start 158.9 121.7) (end 158.8 121.8) (width 0.2) (layer "B.Cu") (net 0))
 (segment (start 126.9 115.28) (end 128.52 115.28) (width 0.2) (layer "B.Cu") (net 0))
 (segment (start 136.3 75) (end 126.7 75) (width 0.2) (layer "B.Cu") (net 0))
 (segment (start 144.8 119) (end 144.8 120.4) (width 0.2) (layer "B.Cu") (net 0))
 (segment (start 149.4 99.5) (end 149.4 99.151) (width 0.2) (layer "B.Cu") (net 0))
 (segment (start 124.2 59.8) (end 124 59.6) (width 0.2) (layer "B.Cu") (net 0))
 (segment (start 124.2 71.8) (end 124.2 64.9) (width 0.2) (layer "B.Cu") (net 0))
 (segment (start 124 59.6) (end 123.6 60) (width 0.2) (layer "B.Cu") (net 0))
 (segment (start 125.36 100.04) (end 126.9 100.04) (width 0.2) (layer "B.Cu") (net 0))
 (segment (start 124.3 71.9) (end 124.2 71.8) (width 0.2) (layer "B.Cu") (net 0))
 (segment (start 158.8 121.8) (end 125.6 121.8) (width 0.2) (layer "B.Cu") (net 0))
 (segment (start 133.1 82.8) (end 133.1 62) (width 0.2) (layer "B.Cu") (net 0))
 (segment (start 152.9 118.3) (end 152.9 82.74) (width 0.2) (layer "B.Cu") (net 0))
 (segment (start 144.8 120.4) (end 155.8 120.4) (width 0.2) (layer "B.Cu") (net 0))
 (segment (start 139.2 59.8) (end 128.94 59.8) (width 0.2) (layer "B.Cu") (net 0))
 (segment (start 158.9 110.68) (end 161.8 113.58) (width 0.2) (layer "B.Cu") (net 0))
 (segment (start 149.4 99.5) (end 149.4 99.2) (width 0.2) (layer "B.Cu") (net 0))
 (segment (start 128.56 112.74) (end 131 110.3) (width 0.2) (layer "B.Cu") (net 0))
 (segment (start 158.9 115.76) (end 160.16 115.76) (width 0.2) (layer "B.Cu") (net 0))
 (segment (start 161.8 124.4) (end 161.5 124.7) (width 0.2) (layer "B.Cu") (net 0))
 (segment (start 136.8 75.5) (end 136.3 75) (width 0.2) (layer "B.Cu") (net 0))
 (segment (start 124.2 64.9) (end 124.22 64.88) (width 0.2) (layer "B.Cu") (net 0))
 (segment (start 139.4 115.3) (end 139.4 59.6) (width 0.2) (layer "B.Cu") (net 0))
 (segment (start 124.8 104.9) (end 125.02 105.12) (width 0.2) (layer "B.Cu") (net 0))
 (segment (start 158.9 118.3) (end 158.9 121.7) (width 0.2) (layer "B.Cu") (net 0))
 (segment (start 138.62 117.82) (end 138.3 117.5) (width 0.2) (layer "B.Cu") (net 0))
 (segment (start 145.4 84.9) (end 145.3 84.8) (width 0.2) (layer "B.Cu") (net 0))
 (segment (start 145.3 84.8) (end 142.14 84.8) (width 0.2) (layer "B.Cu") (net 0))
 (segment (start 136.8 84.5) (end 136.8 75.5) (width 0.2) (layer "B.Cu") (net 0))
 (segment (start 149.449 99.151) (end 149.4 99.151) (width 0.2) (layer "B.Cu") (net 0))
 (segment (start 138 71.9) (end 124.3 71.9) (width 0.2) (layer "B.Cu") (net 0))
 (segment (start 132.8 86) (end 134.9 83.9) (width 0.2) (layer "B.Cu") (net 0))
 (segment (start 144.8 86.9) (end 144.8 86.3) (width 0.2) (layer "B.Cu") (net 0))
 (segment (start 149.4 82.5) (end 149.5 82.4) (width 0.2) (layer "B.Cu") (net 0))
 (segment (start 149.5 82.4) (end 149.36 82.26) (width 0.2) (layer "B.Cu") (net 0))
 (segment (start 146.9 85) (end 146.7 84.8) (width 0.2) (layer "B.Cu") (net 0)))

